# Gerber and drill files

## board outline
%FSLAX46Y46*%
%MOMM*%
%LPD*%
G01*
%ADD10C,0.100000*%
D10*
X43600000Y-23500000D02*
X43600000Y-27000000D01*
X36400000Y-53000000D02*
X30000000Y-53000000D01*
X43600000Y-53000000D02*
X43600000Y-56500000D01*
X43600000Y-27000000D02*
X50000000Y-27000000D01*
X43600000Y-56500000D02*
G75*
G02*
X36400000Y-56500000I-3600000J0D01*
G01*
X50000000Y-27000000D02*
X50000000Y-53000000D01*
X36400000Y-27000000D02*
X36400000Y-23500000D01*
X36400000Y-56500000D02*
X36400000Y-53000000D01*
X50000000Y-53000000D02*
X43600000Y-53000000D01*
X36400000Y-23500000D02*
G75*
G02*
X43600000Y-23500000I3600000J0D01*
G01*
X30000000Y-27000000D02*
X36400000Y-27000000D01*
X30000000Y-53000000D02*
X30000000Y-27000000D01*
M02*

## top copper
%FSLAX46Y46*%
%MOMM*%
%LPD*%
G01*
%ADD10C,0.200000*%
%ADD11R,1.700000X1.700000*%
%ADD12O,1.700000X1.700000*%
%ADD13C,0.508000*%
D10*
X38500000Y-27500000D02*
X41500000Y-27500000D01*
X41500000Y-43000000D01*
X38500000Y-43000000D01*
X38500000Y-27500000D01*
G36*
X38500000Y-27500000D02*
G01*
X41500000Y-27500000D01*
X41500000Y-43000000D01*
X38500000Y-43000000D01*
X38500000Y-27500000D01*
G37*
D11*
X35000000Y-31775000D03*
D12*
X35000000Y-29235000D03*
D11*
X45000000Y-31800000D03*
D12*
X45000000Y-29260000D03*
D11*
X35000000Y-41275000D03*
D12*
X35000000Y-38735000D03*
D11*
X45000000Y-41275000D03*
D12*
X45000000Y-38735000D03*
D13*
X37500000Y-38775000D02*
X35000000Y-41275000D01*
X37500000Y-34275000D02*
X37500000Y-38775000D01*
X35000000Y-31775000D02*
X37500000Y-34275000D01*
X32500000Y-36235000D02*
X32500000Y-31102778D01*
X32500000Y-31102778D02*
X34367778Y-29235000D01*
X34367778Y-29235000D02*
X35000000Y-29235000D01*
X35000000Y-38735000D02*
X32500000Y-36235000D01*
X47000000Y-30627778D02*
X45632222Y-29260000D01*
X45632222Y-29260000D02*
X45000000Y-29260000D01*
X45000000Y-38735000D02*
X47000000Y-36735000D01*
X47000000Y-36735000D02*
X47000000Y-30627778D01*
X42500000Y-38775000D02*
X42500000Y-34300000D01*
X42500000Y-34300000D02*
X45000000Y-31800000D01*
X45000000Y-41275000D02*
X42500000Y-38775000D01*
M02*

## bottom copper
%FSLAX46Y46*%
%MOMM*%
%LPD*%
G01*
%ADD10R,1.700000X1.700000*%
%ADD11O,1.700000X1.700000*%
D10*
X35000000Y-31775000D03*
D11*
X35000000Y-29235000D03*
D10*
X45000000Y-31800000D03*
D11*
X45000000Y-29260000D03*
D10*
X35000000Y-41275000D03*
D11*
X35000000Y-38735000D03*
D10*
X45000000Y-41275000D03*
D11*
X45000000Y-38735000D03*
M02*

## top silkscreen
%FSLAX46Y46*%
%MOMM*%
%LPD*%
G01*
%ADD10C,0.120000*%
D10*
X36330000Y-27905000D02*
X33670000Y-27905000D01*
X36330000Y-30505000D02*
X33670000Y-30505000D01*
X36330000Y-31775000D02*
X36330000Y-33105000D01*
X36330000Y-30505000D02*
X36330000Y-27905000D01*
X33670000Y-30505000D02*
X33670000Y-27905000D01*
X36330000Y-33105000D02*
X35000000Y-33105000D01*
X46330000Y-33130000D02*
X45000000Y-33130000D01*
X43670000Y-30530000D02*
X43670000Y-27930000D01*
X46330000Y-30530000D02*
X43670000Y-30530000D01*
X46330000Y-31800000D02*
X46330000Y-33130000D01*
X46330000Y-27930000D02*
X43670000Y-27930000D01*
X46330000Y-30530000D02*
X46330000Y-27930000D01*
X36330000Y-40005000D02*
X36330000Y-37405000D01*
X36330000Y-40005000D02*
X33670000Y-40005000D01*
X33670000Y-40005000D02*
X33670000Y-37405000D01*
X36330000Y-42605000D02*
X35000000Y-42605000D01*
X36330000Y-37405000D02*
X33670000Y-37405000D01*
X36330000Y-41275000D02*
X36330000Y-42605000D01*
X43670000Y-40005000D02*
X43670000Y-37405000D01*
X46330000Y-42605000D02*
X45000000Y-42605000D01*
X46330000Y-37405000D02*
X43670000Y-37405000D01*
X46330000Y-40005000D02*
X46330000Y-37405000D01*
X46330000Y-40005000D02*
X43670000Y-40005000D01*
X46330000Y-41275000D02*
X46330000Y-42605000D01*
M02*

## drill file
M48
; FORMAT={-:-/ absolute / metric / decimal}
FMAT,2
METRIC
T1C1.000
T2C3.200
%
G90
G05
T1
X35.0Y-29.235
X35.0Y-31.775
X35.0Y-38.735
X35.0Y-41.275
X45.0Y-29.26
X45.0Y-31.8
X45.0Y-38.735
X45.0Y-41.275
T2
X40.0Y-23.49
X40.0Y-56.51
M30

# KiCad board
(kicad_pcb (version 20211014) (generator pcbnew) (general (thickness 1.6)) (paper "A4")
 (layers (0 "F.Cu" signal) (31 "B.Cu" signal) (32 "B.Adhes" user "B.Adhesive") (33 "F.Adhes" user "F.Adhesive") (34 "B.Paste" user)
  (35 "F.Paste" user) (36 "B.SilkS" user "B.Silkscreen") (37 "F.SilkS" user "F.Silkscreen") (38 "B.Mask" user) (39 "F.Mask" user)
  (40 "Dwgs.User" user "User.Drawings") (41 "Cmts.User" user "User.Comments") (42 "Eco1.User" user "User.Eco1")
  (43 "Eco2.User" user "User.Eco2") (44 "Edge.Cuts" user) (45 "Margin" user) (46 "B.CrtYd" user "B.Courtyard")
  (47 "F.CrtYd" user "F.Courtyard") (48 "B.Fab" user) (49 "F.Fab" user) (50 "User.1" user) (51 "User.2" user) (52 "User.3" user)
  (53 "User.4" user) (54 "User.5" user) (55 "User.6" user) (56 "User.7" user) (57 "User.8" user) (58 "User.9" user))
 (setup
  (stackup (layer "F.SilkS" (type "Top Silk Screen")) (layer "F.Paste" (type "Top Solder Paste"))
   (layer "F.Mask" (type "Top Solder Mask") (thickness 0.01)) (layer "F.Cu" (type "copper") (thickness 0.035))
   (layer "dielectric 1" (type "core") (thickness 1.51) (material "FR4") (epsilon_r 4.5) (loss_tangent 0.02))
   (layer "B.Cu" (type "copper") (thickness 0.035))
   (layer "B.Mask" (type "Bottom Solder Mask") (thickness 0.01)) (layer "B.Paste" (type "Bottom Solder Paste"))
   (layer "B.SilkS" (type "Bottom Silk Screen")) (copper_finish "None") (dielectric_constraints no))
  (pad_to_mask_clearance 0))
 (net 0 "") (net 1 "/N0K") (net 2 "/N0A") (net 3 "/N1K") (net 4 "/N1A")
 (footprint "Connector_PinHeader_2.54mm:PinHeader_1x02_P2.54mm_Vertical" (layer "F.Cu") (at 35 31.775 180)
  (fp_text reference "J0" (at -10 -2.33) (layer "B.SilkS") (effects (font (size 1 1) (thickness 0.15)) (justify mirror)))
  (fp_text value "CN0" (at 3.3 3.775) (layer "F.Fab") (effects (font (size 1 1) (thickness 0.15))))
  (fp_line (start -1.33 3.87) (end 1.33 3.87) (layer "F.SilkS") (width 0.12))
  (fp_line (start -1.33 1.27) (end 1.33 1.27) (layer "F.SilkS") (width 0.12))
  (fp_line (start -1.33 0) (end -1.33 -1.33) (layer "F.SilkS") (width 0.12))
  (fp_line (start -1.33 1.27) (end -1.33 3.87) (layer "F.SilkS") (width 0.12))
  (fp_line (start 1.33 1.27) (end 1.33 3.87) (layer "F.SilkS") (width 0.12))
  (fp_line (start -1.33 -1.33) (end 0 -1.33) (layer "F.SilkS") (width 0.12))
  (pad "1" thru_hole rect locked (at 0 0 180) (size 1.7 1.7) (drill 1) (layers *.Cu *.Mask) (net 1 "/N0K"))
  (pad "2" thru_hole oval locked (at 0 2.54 180) (size 1.7 1.7) (drill 1) (layers *.Cu *.Mask) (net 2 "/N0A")))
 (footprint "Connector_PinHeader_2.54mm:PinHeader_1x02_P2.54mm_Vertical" (layer "F.Cu") (at 45 31.8 180)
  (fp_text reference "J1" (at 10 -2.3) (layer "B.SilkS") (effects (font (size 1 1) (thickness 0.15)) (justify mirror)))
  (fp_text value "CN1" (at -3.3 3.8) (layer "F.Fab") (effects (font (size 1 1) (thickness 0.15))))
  (fp_line (start -1.33 -1.33) (end 0 -1.33) (layer "F.SilkS") (width 0.12))
  (fp_line (start 1.33 1.27) (end 1.33 3.87) (layer "F.SilkS") (width 0.12))
  (fp_line (start -1.33 1.27) (end 1.33 1.27) (layer "F.SilkS") (width 0.12))
  (fp_line (start -1.33 0) (end -1.33 -1.33) (layer "F.SilkS") (width 0.12))
  (fp_line (start -1.33 3.87) (end 1.33 3.87) (layer "F.SilkS") (width 0.12))
  (fp_line (start -1.33 1.27) (end -1.33 3.87) (layer "F.SilkS") (width 0.12))
  (pad "1" thru_hole rect locked (at 0 0 180) (size 1.7 1.7) (drill 1) (layers *.Cu *.Mask) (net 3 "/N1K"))
  (pad "2" thru_hole oval locked (at 0 2.54 180) (size 1.7 1.7) (drill 1) (layers *.Cu *.Mask) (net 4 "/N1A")))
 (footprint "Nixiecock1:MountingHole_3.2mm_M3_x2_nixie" (layer "F.Cu") (at 40 40 90)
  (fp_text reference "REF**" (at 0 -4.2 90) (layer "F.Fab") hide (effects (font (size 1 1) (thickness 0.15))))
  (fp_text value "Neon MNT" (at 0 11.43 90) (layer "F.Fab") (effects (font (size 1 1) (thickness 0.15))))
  (pad "" np_thru_hole circle locked (at -16.51 0 90) (size 3.2 3.2) (drill 3.2) (layers *.Cu *.Mask))
  (pad "" np_thru_hole circle locked (at 16.51 0 90) (size 3.2 3.2) (drill 3.2) (layers *.Cu *.Mask)))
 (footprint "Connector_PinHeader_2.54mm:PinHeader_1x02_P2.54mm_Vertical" (layer "F.Cu") (at 35 41.275 180)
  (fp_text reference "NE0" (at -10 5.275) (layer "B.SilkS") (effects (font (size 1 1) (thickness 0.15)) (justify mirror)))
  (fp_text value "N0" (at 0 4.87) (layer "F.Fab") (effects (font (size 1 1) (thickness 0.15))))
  (fp_line (start -1.33 1.27) (end -1.33 3.87) (layer "F.SilkS") (width 0.12))
  (fp_line (start -1.33 1.27) (end 1.33 1.27) (layer "F.SilkS") (width 0.12))
  (fp_line (start 1.33 1.27) (end 1.33 3.87) (layer "F.SilkS") (width 0.12))
  (fp_line (start -1.33 -1.33) (end 0 -1.33) (layer "F.SilkS") (width 0.12))
  (fp_line (start -1.33 3.87) (end 1.33 3.87) (layer "F.SilkS") (width 0.12))
  (fp_line (start -1.33 0) (end -1.33 -1.33) (layer "F.SilkS") (width 0.12))
  (pad "1" thru_hole rect locked (at 0 0 180) (size 1.7 1.7) (drill 1) (layers *.Cu *.Mask) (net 1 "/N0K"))
  (pad "2" thru_hole oval locked (at 0 2.54 180) (size 1.7 1.7) (drill 1) (layers *.Cu *.Mask) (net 2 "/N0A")))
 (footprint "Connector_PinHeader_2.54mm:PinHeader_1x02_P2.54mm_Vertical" (layer "F.Cu") (at 45 41.275 180)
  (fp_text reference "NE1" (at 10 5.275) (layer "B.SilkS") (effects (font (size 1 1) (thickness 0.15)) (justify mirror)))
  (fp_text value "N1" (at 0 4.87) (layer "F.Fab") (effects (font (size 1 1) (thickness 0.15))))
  (fp_line (start 1.33 1.27) (end 1.33 3.87) (layer "F.SilkS") (width 0.12))
  (fp_line (start -1.33 -1.33) (end 0 -1.33) (layer "F.SilkS") (width 0.12))
  (fp_line (start -1.33 3.87) (end 1.33 3.87) (layer "F.SilkS") (width 0.12))
  (fp_line (start -1.33 1.27) (end -1.33 3.87) (layer "F.SilkS") (width 0.12))
  (fp_line (start -1.33 1.27) (end 1.33 1.27) (layer "F.SilkS") (width 0.12))
  (fp_line (start -1.33 0) (end -1.33 -1.33) (layer "F.SilkS") (width 0.12))
  (pad "1" thru_hole rect locked (at 0 0 180) (size 1.7 1.7) (drill 1) (layers *.Cu *.Mask) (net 3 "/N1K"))
  (pad "2" thru_hole oval locked (at 0 2.54 180) (size 1.7 1.7) (drill 1) (layers *.Cu *.Mask) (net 4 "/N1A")))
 (gr_rect (start 38.5 27.5) (end 41.5 43) (layer "F.Cu") (width 0.2) (fill solid))
 (gr_line (start 43.6 23.5) (end 43.6 27) (layer "Edge.Cuts") (width 0.1))
 (gr_line (start 36.4 53) (end 30 53) (layer "Edge.Cuts") (width 0.1))
 (gr_line (start 43.6 53) (end 43.6 56.5) (layer "Edge.Cuts") (width 0.1))
 (gr_line (start 43.6 27) (end 50 27) (layer "Edge.Cuts") (width 0.1))
 (gr_arc (start 43.6 56.5) (mid 40 60.1) (end 36.4 56.5) (layer "Edge.Cuts") (width 0.1))
 (gr_line (start 50 27) (end 50 53) (layer "Edge.Cuts") (width 0.1))
 (gr_line (start 36.4 27) (end 36.4 23.5) (layer "Edge.Cuts") (width 0.1))
 (gr_line (start 36.4 56.5) (end 36.4 53) (layer "Edge.Cuts") (width 0.1))
 (gr_line (start 50 53) (end 43.6 53) (layer "Edge.Cuts") (width 0.1))
 (gr_arc (start 36.4 23.5) (mid 40 19.9) (end 43.6 23.5) (layer "Edge.Cuts") (width 0.1))
 (gr_line (start 30 27) (end 36.4 27) (layer "Edge.Cuts") (width 0.1))
 (gr_line (start 30 53) (end 30 27) (layer "Edge.Cuts") (width 0.1))
 (segment (start 37.5 38.775) (end 35 41.275) (width 0.508) (layer "F.Cu") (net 1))
 (segment (start 37.5 34.275) (end 37.5 38.775) (width 0.508) (layer "F.Cu") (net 1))
 (segment (start 35 31.775) (end 37.5 34.275) (width 0.508) (layer "F.Cu") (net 1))
 (segment (start 32.5 36.235) (end 32.5 31.102778) (width 0.508) (layer "F.Cu") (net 2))
 (segment (start 32.5 31.102778) (end 34.367778 29.235) (width 0.508) (layer "F.Cu") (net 2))
 (segment (start 34.367778 29.235) (end 35 29.235) (width 0.508) (layer "F.Cu") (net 2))
 (segment (start 35 38.735) (end 32.5 36.235) (width 0.508) (layer "F.Cu") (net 2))
 (segment (start 47 30.627778) (end 45.632222 29.26) (width 0.508) (layer "F.Cu") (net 4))
 (segment (start 45.632222 29.26) (end 45 29.26) (width 0.508) (layer "F.Cu") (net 4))
 (segment (start 45 38.735) (end 47 36.735) (width 0.508) (layer "F.Cu") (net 4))
 (segment (start 47 36.735) (end 47 30.627778) (width 0.508) (layer "F.Cu") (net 4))
 (segment (start 42.5 38.775) (end 42.5 34.3) (width 0.508) (layer "F.Cu") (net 3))
 (segment (start 42.5 34.3) (end 45 31.8) (width 0.508) (layer "F.Cu") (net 3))
 (segment (start 45 41.275) (end 42.5 38.775) (width 0.508) (layer "F.Cu") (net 3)))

